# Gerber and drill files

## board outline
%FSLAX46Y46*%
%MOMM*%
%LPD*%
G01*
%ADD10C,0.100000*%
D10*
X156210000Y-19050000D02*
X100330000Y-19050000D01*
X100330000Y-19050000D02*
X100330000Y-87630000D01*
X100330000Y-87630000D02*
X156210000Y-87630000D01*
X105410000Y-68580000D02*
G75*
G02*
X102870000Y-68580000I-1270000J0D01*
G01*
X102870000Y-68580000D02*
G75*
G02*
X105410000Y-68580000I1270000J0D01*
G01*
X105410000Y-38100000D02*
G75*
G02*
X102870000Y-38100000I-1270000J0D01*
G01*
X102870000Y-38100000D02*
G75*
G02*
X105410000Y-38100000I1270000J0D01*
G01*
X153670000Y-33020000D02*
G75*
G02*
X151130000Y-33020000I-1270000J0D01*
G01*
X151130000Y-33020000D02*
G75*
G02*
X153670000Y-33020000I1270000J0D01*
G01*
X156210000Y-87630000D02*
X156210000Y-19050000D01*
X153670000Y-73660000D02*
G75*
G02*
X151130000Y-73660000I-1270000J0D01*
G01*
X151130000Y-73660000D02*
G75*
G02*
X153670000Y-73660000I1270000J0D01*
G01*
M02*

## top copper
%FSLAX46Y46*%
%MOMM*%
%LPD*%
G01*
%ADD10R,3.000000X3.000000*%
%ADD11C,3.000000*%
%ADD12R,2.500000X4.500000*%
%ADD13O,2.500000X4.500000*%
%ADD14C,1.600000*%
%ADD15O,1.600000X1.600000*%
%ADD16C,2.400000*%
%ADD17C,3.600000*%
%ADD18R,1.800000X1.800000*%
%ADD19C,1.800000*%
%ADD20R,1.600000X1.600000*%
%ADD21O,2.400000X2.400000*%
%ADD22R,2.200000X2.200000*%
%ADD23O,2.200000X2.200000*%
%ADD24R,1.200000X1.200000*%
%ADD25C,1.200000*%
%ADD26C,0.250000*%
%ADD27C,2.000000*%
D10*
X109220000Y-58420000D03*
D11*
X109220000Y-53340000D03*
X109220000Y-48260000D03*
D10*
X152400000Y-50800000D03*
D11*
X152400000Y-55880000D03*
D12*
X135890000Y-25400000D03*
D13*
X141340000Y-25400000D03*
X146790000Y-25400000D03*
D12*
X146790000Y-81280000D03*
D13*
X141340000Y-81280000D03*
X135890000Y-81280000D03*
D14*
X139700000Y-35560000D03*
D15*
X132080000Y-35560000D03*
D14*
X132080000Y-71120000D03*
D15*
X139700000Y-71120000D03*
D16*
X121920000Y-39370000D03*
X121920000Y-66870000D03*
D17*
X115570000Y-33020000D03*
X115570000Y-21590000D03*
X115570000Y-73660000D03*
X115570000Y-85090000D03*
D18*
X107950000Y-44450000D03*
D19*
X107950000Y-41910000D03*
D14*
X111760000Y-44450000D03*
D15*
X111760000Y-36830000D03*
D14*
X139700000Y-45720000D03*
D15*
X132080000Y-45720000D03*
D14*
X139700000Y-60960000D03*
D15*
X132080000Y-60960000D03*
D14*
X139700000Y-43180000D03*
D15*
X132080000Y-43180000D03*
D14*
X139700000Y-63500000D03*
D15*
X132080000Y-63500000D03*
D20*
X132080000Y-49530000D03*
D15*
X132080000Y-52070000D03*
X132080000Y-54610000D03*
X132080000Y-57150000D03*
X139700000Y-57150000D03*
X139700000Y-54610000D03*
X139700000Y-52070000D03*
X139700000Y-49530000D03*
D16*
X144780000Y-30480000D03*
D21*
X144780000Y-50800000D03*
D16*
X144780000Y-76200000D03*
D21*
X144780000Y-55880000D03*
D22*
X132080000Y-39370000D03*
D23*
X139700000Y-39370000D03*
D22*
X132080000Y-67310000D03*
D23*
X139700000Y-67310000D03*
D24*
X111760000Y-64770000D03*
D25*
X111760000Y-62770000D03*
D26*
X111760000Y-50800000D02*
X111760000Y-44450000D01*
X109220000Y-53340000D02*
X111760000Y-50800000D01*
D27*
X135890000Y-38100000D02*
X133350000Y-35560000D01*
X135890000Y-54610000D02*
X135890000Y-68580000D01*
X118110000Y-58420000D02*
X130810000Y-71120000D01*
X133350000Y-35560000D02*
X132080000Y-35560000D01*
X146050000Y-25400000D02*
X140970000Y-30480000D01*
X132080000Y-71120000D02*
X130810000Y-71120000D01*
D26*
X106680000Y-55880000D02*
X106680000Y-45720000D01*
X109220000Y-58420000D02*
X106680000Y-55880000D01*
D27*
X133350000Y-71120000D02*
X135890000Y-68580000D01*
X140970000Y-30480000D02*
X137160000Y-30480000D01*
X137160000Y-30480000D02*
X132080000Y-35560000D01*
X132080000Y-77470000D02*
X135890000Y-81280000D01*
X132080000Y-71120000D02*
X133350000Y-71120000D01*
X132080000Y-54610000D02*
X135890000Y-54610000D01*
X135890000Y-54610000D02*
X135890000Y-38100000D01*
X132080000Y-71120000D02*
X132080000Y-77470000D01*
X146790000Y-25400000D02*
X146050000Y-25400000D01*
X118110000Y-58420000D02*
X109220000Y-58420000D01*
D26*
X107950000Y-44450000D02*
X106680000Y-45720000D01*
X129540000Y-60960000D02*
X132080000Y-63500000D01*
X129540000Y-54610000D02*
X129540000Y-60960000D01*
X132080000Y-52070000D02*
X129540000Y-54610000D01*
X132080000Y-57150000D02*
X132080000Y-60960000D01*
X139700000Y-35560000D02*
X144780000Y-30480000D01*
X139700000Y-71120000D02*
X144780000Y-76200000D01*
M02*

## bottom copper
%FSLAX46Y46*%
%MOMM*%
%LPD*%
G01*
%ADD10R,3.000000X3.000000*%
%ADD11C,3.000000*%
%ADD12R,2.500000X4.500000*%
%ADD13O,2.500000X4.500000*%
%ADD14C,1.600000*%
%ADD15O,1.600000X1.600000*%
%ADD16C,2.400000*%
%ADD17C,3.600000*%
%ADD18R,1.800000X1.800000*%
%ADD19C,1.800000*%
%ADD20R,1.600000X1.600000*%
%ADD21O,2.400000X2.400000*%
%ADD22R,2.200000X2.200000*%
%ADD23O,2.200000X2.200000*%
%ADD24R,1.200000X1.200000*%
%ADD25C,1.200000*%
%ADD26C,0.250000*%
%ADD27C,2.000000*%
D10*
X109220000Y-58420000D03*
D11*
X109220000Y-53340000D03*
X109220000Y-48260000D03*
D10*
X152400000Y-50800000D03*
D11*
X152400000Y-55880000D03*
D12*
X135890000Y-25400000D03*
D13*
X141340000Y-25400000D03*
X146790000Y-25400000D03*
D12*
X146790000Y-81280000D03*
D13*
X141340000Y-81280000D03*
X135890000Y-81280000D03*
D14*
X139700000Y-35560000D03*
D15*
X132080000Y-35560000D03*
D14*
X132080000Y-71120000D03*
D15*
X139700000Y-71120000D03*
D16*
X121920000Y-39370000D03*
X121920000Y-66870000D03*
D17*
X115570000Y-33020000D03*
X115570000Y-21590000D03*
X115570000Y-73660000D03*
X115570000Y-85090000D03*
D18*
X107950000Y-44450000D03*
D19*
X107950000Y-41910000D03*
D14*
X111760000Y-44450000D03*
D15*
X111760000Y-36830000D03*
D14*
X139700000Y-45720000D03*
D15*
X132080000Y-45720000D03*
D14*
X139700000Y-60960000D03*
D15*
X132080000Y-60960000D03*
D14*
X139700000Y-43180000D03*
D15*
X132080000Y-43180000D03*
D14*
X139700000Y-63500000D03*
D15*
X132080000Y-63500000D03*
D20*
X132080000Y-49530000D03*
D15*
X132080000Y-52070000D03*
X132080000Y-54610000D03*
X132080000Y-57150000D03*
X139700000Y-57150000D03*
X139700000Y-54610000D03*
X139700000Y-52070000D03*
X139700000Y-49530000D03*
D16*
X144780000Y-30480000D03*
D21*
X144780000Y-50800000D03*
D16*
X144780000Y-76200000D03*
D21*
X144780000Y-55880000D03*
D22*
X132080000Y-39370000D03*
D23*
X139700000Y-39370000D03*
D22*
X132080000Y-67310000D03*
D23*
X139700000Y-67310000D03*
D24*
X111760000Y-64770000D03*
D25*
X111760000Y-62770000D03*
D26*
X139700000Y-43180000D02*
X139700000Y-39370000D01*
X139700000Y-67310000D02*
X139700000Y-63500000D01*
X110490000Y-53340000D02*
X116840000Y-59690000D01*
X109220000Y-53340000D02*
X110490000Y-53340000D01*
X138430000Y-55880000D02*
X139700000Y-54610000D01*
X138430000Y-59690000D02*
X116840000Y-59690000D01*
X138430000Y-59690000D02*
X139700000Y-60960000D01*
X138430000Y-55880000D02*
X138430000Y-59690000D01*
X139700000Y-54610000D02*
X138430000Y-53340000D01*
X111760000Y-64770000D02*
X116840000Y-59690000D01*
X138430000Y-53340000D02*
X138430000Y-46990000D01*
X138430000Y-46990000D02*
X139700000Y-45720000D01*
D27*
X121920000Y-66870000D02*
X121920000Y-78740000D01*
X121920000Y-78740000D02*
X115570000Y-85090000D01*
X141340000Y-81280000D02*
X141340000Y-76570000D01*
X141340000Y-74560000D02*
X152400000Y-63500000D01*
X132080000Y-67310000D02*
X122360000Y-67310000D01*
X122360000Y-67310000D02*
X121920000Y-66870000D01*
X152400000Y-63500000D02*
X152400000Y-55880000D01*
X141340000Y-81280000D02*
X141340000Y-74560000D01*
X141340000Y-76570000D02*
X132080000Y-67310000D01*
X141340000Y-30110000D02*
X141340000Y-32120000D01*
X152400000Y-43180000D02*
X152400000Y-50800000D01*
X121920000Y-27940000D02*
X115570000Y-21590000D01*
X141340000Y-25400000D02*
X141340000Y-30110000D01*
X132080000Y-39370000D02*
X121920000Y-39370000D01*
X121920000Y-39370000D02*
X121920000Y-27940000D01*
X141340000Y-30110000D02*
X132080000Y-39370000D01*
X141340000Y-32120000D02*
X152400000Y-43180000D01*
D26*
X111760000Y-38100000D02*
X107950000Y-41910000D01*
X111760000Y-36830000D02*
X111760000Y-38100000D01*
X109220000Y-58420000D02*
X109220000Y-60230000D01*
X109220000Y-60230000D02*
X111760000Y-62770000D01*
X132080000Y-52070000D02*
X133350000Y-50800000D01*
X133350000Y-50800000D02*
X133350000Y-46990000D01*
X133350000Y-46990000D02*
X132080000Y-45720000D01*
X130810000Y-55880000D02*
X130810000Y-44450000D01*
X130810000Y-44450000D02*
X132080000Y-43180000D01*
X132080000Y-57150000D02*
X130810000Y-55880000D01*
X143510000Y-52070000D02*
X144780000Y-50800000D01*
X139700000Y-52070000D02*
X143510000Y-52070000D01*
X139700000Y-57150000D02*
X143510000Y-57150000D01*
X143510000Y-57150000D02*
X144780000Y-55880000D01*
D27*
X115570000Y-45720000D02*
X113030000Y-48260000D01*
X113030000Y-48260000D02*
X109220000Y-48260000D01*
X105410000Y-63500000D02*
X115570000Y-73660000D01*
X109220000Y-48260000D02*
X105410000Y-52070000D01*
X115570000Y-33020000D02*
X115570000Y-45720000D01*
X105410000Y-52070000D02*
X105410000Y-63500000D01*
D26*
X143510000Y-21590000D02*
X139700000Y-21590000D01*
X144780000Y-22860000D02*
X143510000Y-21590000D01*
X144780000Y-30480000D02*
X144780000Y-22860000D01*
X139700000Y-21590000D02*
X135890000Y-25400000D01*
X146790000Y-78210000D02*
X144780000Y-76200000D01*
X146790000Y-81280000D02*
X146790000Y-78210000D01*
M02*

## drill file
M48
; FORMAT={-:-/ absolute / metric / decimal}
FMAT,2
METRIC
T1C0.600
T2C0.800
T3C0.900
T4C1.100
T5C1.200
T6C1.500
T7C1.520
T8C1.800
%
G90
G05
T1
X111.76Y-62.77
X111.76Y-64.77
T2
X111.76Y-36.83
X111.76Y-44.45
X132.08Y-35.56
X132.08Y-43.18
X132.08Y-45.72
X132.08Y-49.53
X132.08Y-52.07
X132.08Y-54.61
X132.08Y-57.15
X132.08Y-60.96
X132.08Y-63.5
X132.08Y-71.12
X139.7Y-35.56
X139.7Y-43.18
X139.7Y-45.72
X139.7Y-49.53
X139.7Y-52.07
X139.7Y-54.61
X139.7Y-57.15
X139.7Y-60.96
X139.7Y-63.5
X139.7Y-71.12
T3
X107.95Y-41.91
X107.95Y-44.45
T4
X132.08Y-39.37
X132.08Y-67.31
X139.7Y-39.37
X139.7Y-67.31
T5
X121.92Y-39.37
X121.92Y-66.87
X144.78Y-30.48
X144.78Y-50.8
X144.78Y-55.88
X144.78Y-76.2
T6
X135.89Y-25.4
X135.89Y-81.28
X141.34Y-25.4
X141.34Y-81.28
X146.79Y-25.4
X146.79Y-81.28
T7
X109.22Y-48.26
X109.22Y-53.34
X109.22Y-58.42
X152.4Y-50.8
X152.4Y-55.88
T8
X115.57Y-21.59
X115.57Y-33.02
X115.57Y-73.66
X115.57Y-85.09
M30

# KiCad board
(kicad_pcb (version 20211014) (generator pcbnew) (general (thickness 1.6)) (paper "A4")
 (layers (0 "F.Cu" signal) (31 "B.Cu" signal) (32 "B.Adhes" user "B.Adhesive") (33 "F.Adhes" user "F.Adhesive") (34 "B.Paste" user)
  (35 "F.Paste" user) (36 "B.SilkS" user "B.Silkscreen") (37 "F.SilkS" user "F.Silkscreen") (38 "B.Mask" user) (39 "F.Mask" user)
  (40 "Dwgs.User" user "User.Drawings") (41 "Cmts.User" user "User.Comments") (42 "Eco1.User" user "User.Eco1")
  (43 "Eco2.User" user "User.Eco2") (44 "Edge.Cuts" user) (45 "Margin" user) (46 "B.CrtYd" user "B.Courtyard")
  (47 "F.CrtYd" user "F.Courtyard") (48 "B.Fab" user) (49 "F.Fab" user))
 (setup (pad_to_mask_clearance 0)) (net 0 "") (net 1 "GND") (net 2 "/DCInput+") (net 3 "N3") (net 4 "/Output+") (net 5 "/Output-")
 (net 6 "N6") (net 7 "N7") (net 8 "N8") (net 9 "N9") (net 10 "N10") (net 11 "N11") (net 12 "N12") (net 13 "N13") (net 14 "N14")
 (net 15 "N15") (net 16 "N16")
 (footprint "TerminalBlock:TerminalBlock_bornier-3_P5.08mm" (layer "F.Cu") (at 109.22 58.42 90)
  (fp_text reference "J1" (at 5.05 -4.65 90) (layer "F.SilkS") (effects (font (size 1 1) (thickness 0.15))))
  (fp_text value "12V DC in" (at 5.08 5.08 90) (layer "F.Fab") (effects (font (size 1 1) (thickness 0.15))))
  (pad "1" thru_hole rect locked (at 0 0 90) (size 3 3) (drill 1.52) (layers *.Cu *.Mask) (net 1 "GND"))
  (pad "2" thru_hole circle locked (at 5.08 0 90) (size 3 3) (drill 1.52) (layers *.Cu *.Mask) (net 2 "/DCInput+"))
  (pad "3" thru_hole circle locked (at 10.16 0 90) (size 3 3) (drill 1.52) (layers *.Cu *.Mask) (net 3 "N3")))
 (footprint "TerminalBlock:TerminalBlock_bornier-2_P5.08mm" (layer "F.Cu") (at 152.4 50.8 -90)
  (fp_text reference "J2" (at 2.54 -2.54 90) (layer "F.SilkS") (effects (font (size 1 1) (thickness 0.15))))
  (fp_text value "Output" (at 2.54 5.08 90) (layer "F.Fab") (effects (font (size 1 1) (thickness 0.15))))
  (pad "1" thru_hole rect locked (at 0 0 270) (size 3 3) (drill 1.52) (layers *.Cu *.Mask) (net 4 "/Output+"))
  (pad "2" thru_hole circle locked (at 5.08 0 270) (size 3 3) (drill 1.52) (layers *.Cu *.Mask) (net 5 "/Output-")))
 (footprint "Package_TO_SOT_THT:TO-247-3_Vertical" (layer "F.Cu") (at 135.89 25.4)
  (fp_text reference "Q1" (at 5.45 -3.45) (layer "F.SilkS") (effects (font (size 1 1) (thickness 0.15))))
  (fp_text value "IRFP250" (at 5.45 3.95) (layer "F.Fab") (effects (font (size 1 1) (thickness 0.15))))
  (pad "1" thru_hole rect locked (at 0 0) (size 2.5 4.5) (drill 1.5) (layers *.Cu *.Mask) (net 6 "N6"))
  (pad "2" thru_hole oval locked (at 5.45 0) (size 2.5 4.5) (drill 1.5) (layers *.Cu *.Mask) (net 4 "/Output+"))
  (pad "3" thru_hole oval locked (at 10.9 0) (size 2.5 4.5) (drill 1.5) (layers *.Cu *.Mask) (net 1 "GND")))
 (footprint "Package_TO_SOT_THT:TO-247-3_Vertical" (layer "F.Cu") (at 146.79 81.28 180)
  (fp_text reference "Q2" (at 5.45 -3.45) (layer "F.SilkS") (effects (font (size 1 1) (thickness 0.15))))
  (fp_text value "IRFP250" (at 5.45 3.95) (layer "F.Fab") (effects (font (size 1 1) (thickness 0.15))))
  (pad "1" thru_hole rect locked (at 0 0 180) (size 2.5 4.5) (drill 1.5) (layers *.Cu *.Mask) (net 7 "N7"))
  (pad "2" thru_hole oval locked (at 5.45 0 180) (size 2.5 4.5) (drill 1.5) (layers *.Cu *.Mask) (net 5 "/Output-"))
  (pad "3" thru_hole oval locked (at 10.9 0 180) (size 2.5 4.5) (drill 1.5) (layers *.Cu *.Mask) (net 1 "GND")))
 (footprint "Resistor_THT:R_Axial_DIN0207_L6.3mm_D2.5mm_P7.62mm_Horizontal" (layer "F.Cu") (at 139.7 35.56 180)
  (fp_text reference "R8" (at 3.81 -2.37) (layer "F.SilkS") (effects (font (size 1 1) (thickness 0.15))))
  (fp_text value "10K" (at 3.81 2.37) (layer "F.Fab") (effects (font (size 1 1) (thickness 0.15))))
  (pad "1" thru_hole circle locked (at 0 0 180) (size 1.6 1.6) (drill 0.8) (layers *.Cu *.Mask) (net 6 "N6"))
  (pad "2" thru_hole oval locked (at 7.62 0 180) (size 1.6 1.6) (drill 0.8) (layers *.Cu *.Mask) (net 1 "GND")))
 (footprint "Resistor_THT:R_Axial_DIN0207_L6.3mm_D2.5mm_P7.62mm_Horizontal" (layer "F.Cu") (at 132.08 71.12)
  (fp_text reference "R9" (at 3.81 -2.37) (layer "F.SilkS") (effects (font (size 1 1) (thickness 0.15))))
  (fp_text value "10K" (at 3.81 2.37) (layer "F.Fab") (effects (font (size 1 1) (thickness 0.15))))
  (pad "1" thru_hole circle locked (at 0 0) (size 1.6 1.6) (drill 0.8) (layers *.Cu *.Mask) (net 1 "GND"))
  (pad "2" thru_hole oval locked (at 7.62 0) (size 1.6 1.6) (drill 0.8) (layers *.Cu *.Mask) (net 7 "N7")))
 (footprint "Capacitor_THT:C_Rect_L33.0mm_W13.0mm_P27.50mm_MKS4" (layer "F.Cu") (at 121.92 39.37 -90)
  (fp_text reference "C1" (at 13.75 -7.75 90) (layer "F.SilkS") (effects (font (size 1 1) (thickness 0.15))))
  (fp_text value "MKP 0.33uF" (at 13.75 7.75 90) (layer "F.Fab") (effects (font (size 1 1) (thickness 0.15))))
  (pad "1" thru_hole circle locked (at 0 0 270) (size 2.4 2.4) (drill 1.2) (layers *.Cu *.Mask) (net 4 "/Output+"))
  (pad "2" thru_hole circle locked (at 27.5 0 270) (size 2.4 2.4) (drill 1.2) (layers *.Cu *.Mask) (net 5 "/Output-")))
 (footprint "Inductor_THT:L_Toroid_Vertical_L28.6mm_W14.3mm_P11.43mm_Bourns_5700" (layer "F.Cu") (at 115.57 33.02 180)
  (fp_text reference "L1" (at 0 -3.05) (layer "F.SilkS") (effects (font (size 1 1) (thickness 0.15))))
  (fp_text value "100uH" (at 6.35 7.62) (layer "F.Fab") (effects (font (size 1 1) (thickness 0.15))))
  (pad "1" thru_hole circle locked (at 0 0 180) (size 3.6 3.6) (drill 1.8) (layers *.Cu *.Mask) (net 3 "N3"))
  (pad "2" thru_hole circle locked (at 0 11.43 180) (size 3.6 3.6) (drill 1.8) (layers *.Cu *.Mask) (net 4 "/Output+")))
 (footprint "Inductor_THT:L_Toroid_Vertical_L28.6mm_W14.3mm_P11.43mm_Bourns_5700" (layer "F.Cu") (at 115.57 73.66)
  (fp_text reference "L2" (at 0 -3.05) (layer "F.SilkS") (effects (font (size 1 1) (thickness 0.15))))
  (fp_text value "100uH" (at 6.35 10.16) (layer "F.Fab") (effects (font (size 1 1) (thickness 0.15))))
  (pad "1" thru_hole circle locked (at 0 0) (size 3.6 3.6) (drill 1.8) (layers *.Cu *.Mask) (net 3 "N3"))
  (pad "2" thru_hole circle locked (at 0 11.43) (size 3.6 3.6) (drill 1.8) (layers *.Cu *.Mask) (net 5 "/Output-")))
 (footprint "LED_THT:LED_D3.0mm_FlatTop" (layer "F.Cu") (at 107.95 44.45 90)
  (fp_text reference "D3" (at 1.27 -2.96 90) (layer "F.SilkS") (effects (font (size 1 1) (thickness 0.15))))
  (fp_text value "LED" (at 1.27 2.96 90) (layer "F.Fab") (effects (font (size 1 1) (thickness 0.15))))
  (pad "1" thru_hole rect locked (at 0 0 90) (size 1.8 1.8) (drill 0.9) (layers *.Cu *.Mask) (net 1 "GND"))
  (pad "2" thru_hole circle locked (at 2.54 0 90) (size 1.8 1.8) (drill 0.9) (layers *.Cu *.Mask) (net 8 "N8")))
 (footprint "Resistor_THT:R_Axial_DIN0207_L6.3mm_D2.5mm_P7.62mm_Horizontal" (layer "F.Cu") (at 111.76 44.45 90)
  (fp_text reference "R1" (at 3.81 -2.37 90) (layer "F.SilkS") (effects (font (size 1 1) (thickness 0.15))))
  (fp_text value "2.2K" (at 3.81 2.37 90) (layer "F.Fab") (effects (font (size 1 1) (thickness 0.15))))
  (pad "1" thru_hole circle locked (at 0 0 90) (size 1.6 1.6) (drill 0.8) (layers *.Cu *.Mask) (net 2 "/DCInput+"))
  (pad "2" thru_hole oval locked (at 7.62 0 90) (size 1.6 1.6) (drill 0.8) (layers *.Cu *.Mask) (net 8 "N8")))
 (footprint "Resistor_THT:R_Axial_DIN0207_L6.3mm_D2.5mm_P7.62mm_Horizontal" (layer "F.Cu") (at 139.7 45.72 180)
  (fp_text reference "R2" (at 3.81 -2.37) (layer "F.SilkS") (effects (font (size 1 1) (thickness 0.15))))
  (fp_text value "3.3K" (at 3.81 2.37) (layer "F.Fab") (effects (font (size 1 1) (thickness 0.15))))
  (pad "1" thru_hole circle locked (at 0 0 180) (size 1.6 1.6) (drill 0.8) (layers *.Cu *.Mask) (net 2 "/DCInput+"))
  (pad "2" thru_hole oval locked (at 7.62 0 180) (size 1.6 1.6) (drill 0.8) (layers *.Cu *.Mask) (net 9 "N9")))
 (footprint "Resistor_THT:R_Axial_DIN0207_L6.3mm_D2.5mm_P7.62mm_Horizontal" (layer "F.Cu") (at 139.7 60.96 180)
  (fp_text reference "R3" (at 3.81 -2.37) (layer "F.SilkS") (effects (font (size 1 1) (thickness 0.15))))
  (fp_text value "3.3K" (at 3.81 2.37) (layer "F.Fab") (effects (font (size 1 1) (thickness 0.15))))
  (pad "1" thru_hole circle locked (at 0 0 180) (size 1.6 1.6) (drill 0.8) (layers *.Cu *.Mask) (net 2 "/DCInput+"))
  (pad "2" thru_hole oval locked (at 7.62 0 180) (size 1.6 1.6) (drill 0.8) (layers *.Cu *.Mask) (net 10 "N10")))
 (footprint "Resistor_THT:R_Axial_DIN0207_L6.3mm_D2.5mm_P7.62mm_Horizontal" (layer "F.Cu") (at 139.7 43.18 180)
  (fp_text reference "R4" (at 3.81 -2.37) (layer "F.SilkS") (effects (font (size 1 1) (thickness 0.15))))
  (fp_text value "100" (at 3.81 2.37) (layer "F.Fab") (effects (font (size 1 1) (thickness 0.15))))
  (pad "1" thru_hole circle locked (at 0 0 180) (size 1.6 1.6) (drill 0.8) (layers *.Cu *.Mask) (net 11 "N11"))
  (pad "2" thru_hole oval locked (at 7.62 0 180) (size 1.6 1.6) (drill 0.8) (layers *.Cu *.Mask) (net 10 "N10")))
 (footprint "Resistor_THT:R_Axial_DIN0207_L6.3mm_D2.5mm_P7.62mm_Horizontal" (layer "F.Cu") (at 139.7 63.5 180)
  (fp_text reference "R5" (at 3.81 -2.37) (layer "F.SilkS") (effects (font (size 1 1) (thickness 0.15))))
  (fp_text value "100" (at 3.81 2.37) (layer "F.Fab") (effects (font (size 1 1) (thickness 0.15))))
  (pad "1" thru_hole circle locked (at 0 0 180) (size 1.6 1.6) (drill 0.8) (layers *.Cu *.Mask) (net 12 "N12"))
  (pad "2" thru_hole oval locked (at 7.62 0 180) (size 1.6 1.6) (drill 0.8) (layers *.Cu *.Mask) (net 9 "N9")))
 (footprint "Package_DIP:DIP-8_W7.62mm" (layer "F.Cu") (at 132.08 49.53)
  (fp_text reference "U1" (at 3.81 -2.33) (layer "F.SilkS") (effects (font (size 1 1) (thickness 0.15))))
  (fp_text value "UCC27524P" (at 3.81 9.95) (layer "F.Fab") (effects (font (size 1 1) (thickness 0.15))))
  (pad "1" thru_hole rect locked (at 0 0) (size 1.6 1.6) (drill 0.8) (layers *.Cu *.Mask) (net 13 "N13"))
  (pad "2" thru_hole oval locked (at 0 2.54) (size 1.6 1.6) (drill 0.8) (layers *.Cu *.Mask) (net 9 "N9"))
  (pad "3" thru_hole oval locked (at 0 5.08) (size 1.6 1.6) (drill 0.8) (layers *.Cu *.Mask) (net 1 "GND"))
  (pad "4" thru_hole oval locked (at 0 7.62) (size 1.6 1.6) (drill 0.8) (layers *.Cu *.Mask) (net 10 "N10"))
  (pad "5" thru_hole oval locked (at 7.62 7.62) (size 1.6 1.6) (drill 0.8) (layers *.Cu *.Mask) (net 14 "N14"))
  (pad "6" thru_hole oval locked (at 7.62 5.08) (size 1.6 1.6) (drill 0.8) (layers *.Cu *.Mask) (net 2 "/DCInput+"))
  (pad "7" thru_hole oval locked (at 7.62 2.54) (size 1.6 1.6) (drill 0.8) (layers *.Cu *.Mask) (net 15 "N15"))
  (pad "8" thru_hole oval locked (at 7.62 0) (size 1.6 1.6) (drill 0.8) (layers *.Cu *.Mask) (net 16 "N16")))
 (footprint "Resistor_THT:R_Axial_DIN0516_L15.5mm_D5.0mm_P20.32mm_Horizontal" (layer "F.Cu") (at 144.78 30.48 -90)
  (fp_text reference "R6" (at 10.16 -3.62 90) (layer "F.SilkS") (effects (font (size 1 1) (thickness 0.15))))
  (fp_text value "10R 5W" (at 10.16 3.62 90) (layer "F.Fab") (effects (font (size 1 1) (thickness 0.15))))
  (pad "1" thru_hole circle locked (at 0 0 270) (size 2.4 2.4) (drill 1.2) (layers *.Cu *.Mask) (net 6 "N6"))
  (pad "2" thru_hole oval locked (at 20.32 0 270) (size 2.4 2.4) (drill 1.2) (layers *.Cu *.Mask) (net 15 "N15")))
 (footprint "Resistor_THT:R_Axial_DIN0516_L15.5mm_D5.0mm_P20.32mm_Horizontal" (layer "F.Cu") (at 144.78 76.2 90)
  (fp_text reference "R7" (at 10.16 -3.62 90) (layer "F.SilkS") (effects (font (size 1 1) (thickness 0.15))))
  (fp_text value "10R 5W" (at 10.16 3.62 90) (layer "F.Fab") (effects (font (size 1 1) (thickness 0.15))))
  (pad "1" thru_hole circle locked (at 0 0 90) (size 2.4 2.4) (drill 1.2) (layers *.Cu *.Mask) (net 7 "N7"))
  (pad "2" thru_hole oval locked (at 20.32 0 90) (size 2.4 2.4) (drill 1.2) (layers *.Cu *.Mask) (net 14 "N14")))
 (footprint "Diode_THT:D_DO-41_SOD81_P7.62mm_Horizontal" (layer "F.Cu") (at 132.08 39.37)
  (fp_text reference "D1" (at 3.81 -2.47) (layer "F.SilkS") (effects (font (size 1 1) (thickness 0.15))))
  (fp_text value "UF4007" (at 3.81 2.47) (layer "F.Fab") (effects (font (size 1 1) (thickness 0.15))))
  (pad "1" thru_hole rect locked (at 0 0) (size 2.2 2.2) (drill 1.1) (layers *.Cu *.Mask) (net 4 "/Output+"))
  (pad "2" thru_hole oval locked (at 7.62 0) (size 2.2 2.2) (drill 1.1) (layers *.Cu *.Mask) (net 11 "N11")))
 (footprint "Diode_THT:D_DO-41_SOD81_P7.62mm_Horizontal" (layer "F.Cu") (at 132.08 67.31)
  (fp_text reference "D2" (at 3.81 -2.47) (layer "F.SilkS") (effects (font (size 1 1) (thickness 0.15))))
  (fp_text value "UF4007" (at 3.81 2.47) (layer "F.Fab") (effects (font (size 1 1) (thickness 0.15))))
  (pad "1" thru_hole rect locked (at 0 0) (size 2.2 2.2) (drill 1.1) (layers *.Cu *.Mask) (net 5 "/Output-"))
  (pad "2" thru_hole oval locked (at 7.62 0) (size 2.2 2.2) (drill 1.1) (layers *.Cu *.Mask) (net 12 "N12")))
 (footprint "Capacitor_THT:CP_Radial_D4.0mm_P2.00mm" (layer "F.Cu") (at 111.76 64.77 90)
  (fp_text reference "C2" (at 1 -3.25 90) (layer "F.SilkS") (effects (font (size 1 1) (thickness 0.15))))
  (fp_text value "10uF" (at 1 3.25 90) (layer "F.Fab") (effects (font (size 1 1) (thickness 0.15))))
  (pad "1" thru_hole rect locked (at 0 0 90) (size 1.2 1.2) (drill 0.6) (layers *.Cu *.Mask) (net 2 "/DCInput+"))
  (pad "2" thru_hole circle locked (at 2 0 90) (size 1.2 1.2) (drill 0.6) (layers *.Cu *.Mask) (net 1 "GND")))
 (gr_line (start 156.21 19.05) (end 100.33 19.05) (layer "Edge.Cuts") (width 0.1))
 (gr_line (start 100.33 19.05) (end 100.33 87.63) (layer "Edge.Cuts") (width 0.1))
 (gr_line (start 100.33 87.63) (end 156.21 87.63) (layer "Edge.Cuts") (width 0.1))
 (gr_circle (center 104.14 68.58) (end 102.87 68.58) (layer "Edge.Cuts") (width 0.1) (fill none))
 (gr_circle (center 104.14 38.1) (end 102.87 38.1) (layer "Edge.Cuts") (width 0.1) (fill none))
 (gr_circle (center 152.4 33.02) (end 153.67 33.02) (layer "Edge.Cuts") (width 0.1) (fill none))
 (gr_line (start 156.21 87.63) (end 156.21 19.05) (layer "Edge.Cuts") (width 0.1))
 (gr_circle (center 152.4 73.66) (end 153.67 73.66) (layer "Edge.Cuts") (width 0.1) (fill none))
 (segment (start 139.7 43.18) (end 139.7 39.37) (width 0.25) (layer "B.Cu") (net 11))
 (segment (start 139.7 67.31) (end 139.7 63.5) (width 0.25) (layer "B.Cu") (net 12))
 (segment (start 111.76 50.8) (end 111.76 44.45) (width 0.25) (layer "F.Cu") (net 2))
 (segment (start 109.22 53.34) (end 111.76 50.8) (width 0.25) (layer "F.Cu") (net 2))
 (segment (start 110.49 53.34) (end 116.84 59.69) (width 0.25) (layer "B.Cu") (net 2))
 (segment (start 109.22 53.34) (end 110.49 53.34) (width 0.25) (layer "B.Cu") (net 2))
 (segment (start 138.43 55.88) (end 139.7 54.61) (width 0.25) (layer "B.Cu") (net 2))
 (segment (start 138.43 59.69) (end 116.84 59.69) (width 0.25) (layer "B.Cu") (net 2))
 (segment (start 138.43 59.69) (end 139.7 60.96) (width 0.25) (layer "B.Cu") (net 2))
 (segment (start 138.43 55.88) (end 138.43 59.69) (width 0.25) (layer "B.Cu") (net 2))
 (segment (start 139.7 54.61) (end 138.43 53.34) (width 0.25) (layer "B.Cu") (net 2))
 (segment (start 111.76 64.77) (end 116.84 59.69) (width 0.25) (layer "B.Cu") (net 2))
 (segment (start 138.43 53.34) (end 138.43 46.99) (width 0.25) (layer "B.Cu") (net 2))
 (segment (start 138.43 46.99) (end 139.7 45.72) (width 0.25) (layer "B.Cu") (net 2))
 (segment (start 121.92 66.87) (end 121.92 78.74) (width 2) (layer "B.Cu") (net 5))
 (segment (start 121.92 78.74) (end 115.57 85.09) (width 2) (layer "B.Cu") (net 5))
 (segment (start 141.34 81.28) (end 141.34 76.57) (width 2) (layer "B.Cu") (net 5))
 (segment (start 141.34 74.56) (end 152.4 63.5) (width 2) (layer "B.Cu") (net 5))
 (segment (start 132.08 67.31) (end 122.36 67.31) (width 2) (layer "B.Cu") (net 5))
 (segment (start 122.36 67.31) (end 121.92 66.87) (width 2) (layer "B.Cu") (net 5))
 (segment (start 152.4 63.5) (end 152.4 55.88) (width 2) (layer "B.Cu") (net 5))
 (segment (start 141.34 81.28) (end 141.34 74.56) (width 2) (layer "B.Cu") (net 5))
 (segment (start 141.34 76.57) (end 132.08 67.31) (width 2) (layer "B.Cu") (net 5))
 (segment (start 141.34 30.11) (end 141.34 32.12) (width 2) (layer "B.Cu") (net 4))
 (segment (start 152.4 43.18) (end 152.4 50.8) (width 2) (layer "B.Cu") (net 4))
 (segment (start 121.92 27.94) (end 115.57 21.59) (width 2) (layer "B.Cu") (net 4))
 (segment (start 141.34 25.4) (end 141.34 30.11) (width 2) (layer "B.Cu") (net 4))
 (segment (start 132.08 39.37) (end 121.92 39.37) (width 2) (layer "B.Cu") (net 4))
 (segment (start 121.92 39.37) (end 121.92 27.94) (width 2) (layer "B.Cu") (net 4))
 (segment (start 141.34 30.11) (end 132.08 39.37) (width 2) (layer "B.Cu") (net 4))
 (segment (start 141.34 32.12) (end 152.4 43.18) (width 2) (layer "B.Cu") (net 4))
 (segment (start 111.76 38.1) (end 107.95 41.91) (width 0.25) (layer "B.Cu") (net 8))
 (segment (start 111.76 36.83) (end 111.76 38.1) (width 0.25) (layer "B.Cu") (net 8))
 (segment (start 135.89 38.1) (end 133.35 35.56) (width 2) (layer "F.Cu") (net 1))
 (segment (start 135.89 54.61) (end 135.89 68.58) (width 2) (layer "F.Cu") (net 1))
 (segment (start 118.11 58.42) (end 130.81 71.12) (width 2) (layer "F.Cu") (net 1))
 (segment (start 133.35 35.56) (end 132.08 35.56) (width 2) (layer "F.Cu") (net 1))
 (segment (start 146.05 25.4) (end 140.97 30.48) (width 2) (layer "F.Cu") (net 1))
 (segment (start 132.08 71.12) (end 130.81 71.12) (width 2) (layer "F.Cu") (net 1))
 (segment (start 106.68 55.88) (end 106.68 45.72) (width 0.25) (layer "F.Cu") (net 1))
 (segment (start 109.22 58.42) (end 106.68 55.88) (width 0.25) (layer "F.Cu") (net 1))
 (segment (start 133.35 71.12) (end 135.89 68.58) (width 2) (layer "F.Cu") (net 1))
 (segment (start 140.97 30.48) (end 137.16 30.48) (width 2) (layer "F.Cu") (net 1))
 (segment (start 137.16 30.48) (end 132.08 35.56) (width 2) (layer "F.Cu") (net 1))
 (segment (start 132.08 77.47) (end 135.89 81.28) (width 2) (layer "F.Cu") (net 1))
 (segment (start 132.08 71.12) (end 133.35 71.12) (width 2) (layer "F.Cu") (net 1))
 (segment (start 132.08 54.61) (end 135.89 54.61) (width 2) (layer "F.Cu") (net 1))
 (segment (start 135.89 54.61) (end 135.89 38.1) (width 2) (layer "F.Cu") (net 1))
 (segment (start 132.08 71.12) (end 132.08 77.47) (width 2) (layer "F.Cu") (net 1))
 (segment (start 146.79 25.4) (end 146.05 25.4) (width 2) (layer "F.Cu") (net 1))
 (segment (start 118.11 58.42) (end 109.22 58.42) (width 2) (layer "F.Cu") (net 1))
 (segment (start 107.95 44.45) (end 106.68 45.72) (width 0.25) (layer "F.Cu") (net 1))
 (segment (start 109.22 58.42) (end 109.22 60.23) (width 0.25) (layer "B.Cu") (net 1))
 (segment (start 109.22 60.23) (end 111.76 62.77) (width 0.25) (layer "B.Cu") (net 1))
 (segment (start 129.54 60.96) (end 132.08 63.5) (width 0.25) (layer "F.Cu") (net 9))
 (segment (start 129.54 54.61) (end 129.54 60.96) (width 0.25) (layer "F.Cu") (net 9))
 (segment (start 132.08 52.07) (end 129.54 54.61) (width 0.25) (layer "F.Cu") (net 9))
 (segment (start 132.08 52.07) (end 133.35 50.8) (width 0.25) (layer "B.Cu") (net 9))
 (segment (start 133.35 50.8) (end 133.35 46.99) (width 0.25) (layer "B.Cu") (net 9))
 (segment (start 133.35 46.99) (end 132.08 45.72) (width 0.25) (layer "B.Cu") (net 9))
 (segment (start 132.08 57.15) (end 132.08 60.96) (width 0.25) (layer "F.Cu") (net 10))
 (segment (start 130.81 55.88) (end 130.81 44.45) (width 0.25) (layer "B.Cu") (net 10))
 (segment (start 130.81 44.45) (end 132.08 43.18) (width 0.25) (layer "B.Cu") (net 10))
 (segment (start 132.08 57.15) (end 130.81 55.88) (width 0.25) (layer "B.Cu") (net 10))
 (segment (start 143.51 52.07) (end 144.78 50.8) (width 0.25) (layer "B.Cu") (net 15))
 (segment (start 139.7 52.07) (end 143.51 52.07) (width 0.25) (layer "B.Cu") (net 15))
 (segment (start 139.7 57.15) (end 143.51 57.15) (width 0.25) (layer "B.Cu") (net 14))
 (segment (start 143.51 57.15) (end 144.78 55.88) (width 0.25) (layer "B.Cu") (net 14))
 (segment (start 115.57 45.72) (end 113.03 48.26) (width 2) (layer "B.Cu") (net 3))
 (segment (start 113.03 48.26) (end 109.22 48.26) (width 2) (layer "B.Cu") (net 3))
 (segment (start 105.41 63.5) (end 115.57 73.66) (width 2) (layer "B.Cu") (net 3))
 (segment (start 109.22 48.26) (end 105.41 52.07) (width 2) (layer "B.Cu") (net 3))
 (segment (start 115.57 33.02) (end 115.57 45.72) (width 2) (layer "B.Cu") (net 3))
 (segment (start 105.41 52.07) (end 105.41 63.5) (width 2) (layer "B.Cu") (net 3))
 (segment (start 139.7 35.56) (end 144.78 30.48) (width 0.25) (layer "F.Cu") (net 6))
 (segment (start 143.51 21.59) (end 139.7 21.59) (width 0.25) (layer "B.Cu") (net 6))
 (segment (start 144.78 22.86) (end 143.51 21.59) (width 0.25) (layer "B.Cu") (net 6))
 (segment (start 144.78 30.48) (end 144.78 22.86) (width 0.25) (layer "B.Cu") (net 6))
 (segment (start 139.7 21.59) (end 135.89 25.4) (width 0.25) (layer "B.Cu") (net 6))
 (segment (start 139.7 71.12) (end 144.78 76.2) (width 0.25) (layer "F.Cu") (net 7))
 (segment (start 146.79 78.21) (end 144.78 76.2) (width 0.25) (layer "B.Cu") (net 7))
 (segment (start 146.79 81.28) (end 146.79 78.21) (width 0.25) (layer "B.Cu") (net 7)))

